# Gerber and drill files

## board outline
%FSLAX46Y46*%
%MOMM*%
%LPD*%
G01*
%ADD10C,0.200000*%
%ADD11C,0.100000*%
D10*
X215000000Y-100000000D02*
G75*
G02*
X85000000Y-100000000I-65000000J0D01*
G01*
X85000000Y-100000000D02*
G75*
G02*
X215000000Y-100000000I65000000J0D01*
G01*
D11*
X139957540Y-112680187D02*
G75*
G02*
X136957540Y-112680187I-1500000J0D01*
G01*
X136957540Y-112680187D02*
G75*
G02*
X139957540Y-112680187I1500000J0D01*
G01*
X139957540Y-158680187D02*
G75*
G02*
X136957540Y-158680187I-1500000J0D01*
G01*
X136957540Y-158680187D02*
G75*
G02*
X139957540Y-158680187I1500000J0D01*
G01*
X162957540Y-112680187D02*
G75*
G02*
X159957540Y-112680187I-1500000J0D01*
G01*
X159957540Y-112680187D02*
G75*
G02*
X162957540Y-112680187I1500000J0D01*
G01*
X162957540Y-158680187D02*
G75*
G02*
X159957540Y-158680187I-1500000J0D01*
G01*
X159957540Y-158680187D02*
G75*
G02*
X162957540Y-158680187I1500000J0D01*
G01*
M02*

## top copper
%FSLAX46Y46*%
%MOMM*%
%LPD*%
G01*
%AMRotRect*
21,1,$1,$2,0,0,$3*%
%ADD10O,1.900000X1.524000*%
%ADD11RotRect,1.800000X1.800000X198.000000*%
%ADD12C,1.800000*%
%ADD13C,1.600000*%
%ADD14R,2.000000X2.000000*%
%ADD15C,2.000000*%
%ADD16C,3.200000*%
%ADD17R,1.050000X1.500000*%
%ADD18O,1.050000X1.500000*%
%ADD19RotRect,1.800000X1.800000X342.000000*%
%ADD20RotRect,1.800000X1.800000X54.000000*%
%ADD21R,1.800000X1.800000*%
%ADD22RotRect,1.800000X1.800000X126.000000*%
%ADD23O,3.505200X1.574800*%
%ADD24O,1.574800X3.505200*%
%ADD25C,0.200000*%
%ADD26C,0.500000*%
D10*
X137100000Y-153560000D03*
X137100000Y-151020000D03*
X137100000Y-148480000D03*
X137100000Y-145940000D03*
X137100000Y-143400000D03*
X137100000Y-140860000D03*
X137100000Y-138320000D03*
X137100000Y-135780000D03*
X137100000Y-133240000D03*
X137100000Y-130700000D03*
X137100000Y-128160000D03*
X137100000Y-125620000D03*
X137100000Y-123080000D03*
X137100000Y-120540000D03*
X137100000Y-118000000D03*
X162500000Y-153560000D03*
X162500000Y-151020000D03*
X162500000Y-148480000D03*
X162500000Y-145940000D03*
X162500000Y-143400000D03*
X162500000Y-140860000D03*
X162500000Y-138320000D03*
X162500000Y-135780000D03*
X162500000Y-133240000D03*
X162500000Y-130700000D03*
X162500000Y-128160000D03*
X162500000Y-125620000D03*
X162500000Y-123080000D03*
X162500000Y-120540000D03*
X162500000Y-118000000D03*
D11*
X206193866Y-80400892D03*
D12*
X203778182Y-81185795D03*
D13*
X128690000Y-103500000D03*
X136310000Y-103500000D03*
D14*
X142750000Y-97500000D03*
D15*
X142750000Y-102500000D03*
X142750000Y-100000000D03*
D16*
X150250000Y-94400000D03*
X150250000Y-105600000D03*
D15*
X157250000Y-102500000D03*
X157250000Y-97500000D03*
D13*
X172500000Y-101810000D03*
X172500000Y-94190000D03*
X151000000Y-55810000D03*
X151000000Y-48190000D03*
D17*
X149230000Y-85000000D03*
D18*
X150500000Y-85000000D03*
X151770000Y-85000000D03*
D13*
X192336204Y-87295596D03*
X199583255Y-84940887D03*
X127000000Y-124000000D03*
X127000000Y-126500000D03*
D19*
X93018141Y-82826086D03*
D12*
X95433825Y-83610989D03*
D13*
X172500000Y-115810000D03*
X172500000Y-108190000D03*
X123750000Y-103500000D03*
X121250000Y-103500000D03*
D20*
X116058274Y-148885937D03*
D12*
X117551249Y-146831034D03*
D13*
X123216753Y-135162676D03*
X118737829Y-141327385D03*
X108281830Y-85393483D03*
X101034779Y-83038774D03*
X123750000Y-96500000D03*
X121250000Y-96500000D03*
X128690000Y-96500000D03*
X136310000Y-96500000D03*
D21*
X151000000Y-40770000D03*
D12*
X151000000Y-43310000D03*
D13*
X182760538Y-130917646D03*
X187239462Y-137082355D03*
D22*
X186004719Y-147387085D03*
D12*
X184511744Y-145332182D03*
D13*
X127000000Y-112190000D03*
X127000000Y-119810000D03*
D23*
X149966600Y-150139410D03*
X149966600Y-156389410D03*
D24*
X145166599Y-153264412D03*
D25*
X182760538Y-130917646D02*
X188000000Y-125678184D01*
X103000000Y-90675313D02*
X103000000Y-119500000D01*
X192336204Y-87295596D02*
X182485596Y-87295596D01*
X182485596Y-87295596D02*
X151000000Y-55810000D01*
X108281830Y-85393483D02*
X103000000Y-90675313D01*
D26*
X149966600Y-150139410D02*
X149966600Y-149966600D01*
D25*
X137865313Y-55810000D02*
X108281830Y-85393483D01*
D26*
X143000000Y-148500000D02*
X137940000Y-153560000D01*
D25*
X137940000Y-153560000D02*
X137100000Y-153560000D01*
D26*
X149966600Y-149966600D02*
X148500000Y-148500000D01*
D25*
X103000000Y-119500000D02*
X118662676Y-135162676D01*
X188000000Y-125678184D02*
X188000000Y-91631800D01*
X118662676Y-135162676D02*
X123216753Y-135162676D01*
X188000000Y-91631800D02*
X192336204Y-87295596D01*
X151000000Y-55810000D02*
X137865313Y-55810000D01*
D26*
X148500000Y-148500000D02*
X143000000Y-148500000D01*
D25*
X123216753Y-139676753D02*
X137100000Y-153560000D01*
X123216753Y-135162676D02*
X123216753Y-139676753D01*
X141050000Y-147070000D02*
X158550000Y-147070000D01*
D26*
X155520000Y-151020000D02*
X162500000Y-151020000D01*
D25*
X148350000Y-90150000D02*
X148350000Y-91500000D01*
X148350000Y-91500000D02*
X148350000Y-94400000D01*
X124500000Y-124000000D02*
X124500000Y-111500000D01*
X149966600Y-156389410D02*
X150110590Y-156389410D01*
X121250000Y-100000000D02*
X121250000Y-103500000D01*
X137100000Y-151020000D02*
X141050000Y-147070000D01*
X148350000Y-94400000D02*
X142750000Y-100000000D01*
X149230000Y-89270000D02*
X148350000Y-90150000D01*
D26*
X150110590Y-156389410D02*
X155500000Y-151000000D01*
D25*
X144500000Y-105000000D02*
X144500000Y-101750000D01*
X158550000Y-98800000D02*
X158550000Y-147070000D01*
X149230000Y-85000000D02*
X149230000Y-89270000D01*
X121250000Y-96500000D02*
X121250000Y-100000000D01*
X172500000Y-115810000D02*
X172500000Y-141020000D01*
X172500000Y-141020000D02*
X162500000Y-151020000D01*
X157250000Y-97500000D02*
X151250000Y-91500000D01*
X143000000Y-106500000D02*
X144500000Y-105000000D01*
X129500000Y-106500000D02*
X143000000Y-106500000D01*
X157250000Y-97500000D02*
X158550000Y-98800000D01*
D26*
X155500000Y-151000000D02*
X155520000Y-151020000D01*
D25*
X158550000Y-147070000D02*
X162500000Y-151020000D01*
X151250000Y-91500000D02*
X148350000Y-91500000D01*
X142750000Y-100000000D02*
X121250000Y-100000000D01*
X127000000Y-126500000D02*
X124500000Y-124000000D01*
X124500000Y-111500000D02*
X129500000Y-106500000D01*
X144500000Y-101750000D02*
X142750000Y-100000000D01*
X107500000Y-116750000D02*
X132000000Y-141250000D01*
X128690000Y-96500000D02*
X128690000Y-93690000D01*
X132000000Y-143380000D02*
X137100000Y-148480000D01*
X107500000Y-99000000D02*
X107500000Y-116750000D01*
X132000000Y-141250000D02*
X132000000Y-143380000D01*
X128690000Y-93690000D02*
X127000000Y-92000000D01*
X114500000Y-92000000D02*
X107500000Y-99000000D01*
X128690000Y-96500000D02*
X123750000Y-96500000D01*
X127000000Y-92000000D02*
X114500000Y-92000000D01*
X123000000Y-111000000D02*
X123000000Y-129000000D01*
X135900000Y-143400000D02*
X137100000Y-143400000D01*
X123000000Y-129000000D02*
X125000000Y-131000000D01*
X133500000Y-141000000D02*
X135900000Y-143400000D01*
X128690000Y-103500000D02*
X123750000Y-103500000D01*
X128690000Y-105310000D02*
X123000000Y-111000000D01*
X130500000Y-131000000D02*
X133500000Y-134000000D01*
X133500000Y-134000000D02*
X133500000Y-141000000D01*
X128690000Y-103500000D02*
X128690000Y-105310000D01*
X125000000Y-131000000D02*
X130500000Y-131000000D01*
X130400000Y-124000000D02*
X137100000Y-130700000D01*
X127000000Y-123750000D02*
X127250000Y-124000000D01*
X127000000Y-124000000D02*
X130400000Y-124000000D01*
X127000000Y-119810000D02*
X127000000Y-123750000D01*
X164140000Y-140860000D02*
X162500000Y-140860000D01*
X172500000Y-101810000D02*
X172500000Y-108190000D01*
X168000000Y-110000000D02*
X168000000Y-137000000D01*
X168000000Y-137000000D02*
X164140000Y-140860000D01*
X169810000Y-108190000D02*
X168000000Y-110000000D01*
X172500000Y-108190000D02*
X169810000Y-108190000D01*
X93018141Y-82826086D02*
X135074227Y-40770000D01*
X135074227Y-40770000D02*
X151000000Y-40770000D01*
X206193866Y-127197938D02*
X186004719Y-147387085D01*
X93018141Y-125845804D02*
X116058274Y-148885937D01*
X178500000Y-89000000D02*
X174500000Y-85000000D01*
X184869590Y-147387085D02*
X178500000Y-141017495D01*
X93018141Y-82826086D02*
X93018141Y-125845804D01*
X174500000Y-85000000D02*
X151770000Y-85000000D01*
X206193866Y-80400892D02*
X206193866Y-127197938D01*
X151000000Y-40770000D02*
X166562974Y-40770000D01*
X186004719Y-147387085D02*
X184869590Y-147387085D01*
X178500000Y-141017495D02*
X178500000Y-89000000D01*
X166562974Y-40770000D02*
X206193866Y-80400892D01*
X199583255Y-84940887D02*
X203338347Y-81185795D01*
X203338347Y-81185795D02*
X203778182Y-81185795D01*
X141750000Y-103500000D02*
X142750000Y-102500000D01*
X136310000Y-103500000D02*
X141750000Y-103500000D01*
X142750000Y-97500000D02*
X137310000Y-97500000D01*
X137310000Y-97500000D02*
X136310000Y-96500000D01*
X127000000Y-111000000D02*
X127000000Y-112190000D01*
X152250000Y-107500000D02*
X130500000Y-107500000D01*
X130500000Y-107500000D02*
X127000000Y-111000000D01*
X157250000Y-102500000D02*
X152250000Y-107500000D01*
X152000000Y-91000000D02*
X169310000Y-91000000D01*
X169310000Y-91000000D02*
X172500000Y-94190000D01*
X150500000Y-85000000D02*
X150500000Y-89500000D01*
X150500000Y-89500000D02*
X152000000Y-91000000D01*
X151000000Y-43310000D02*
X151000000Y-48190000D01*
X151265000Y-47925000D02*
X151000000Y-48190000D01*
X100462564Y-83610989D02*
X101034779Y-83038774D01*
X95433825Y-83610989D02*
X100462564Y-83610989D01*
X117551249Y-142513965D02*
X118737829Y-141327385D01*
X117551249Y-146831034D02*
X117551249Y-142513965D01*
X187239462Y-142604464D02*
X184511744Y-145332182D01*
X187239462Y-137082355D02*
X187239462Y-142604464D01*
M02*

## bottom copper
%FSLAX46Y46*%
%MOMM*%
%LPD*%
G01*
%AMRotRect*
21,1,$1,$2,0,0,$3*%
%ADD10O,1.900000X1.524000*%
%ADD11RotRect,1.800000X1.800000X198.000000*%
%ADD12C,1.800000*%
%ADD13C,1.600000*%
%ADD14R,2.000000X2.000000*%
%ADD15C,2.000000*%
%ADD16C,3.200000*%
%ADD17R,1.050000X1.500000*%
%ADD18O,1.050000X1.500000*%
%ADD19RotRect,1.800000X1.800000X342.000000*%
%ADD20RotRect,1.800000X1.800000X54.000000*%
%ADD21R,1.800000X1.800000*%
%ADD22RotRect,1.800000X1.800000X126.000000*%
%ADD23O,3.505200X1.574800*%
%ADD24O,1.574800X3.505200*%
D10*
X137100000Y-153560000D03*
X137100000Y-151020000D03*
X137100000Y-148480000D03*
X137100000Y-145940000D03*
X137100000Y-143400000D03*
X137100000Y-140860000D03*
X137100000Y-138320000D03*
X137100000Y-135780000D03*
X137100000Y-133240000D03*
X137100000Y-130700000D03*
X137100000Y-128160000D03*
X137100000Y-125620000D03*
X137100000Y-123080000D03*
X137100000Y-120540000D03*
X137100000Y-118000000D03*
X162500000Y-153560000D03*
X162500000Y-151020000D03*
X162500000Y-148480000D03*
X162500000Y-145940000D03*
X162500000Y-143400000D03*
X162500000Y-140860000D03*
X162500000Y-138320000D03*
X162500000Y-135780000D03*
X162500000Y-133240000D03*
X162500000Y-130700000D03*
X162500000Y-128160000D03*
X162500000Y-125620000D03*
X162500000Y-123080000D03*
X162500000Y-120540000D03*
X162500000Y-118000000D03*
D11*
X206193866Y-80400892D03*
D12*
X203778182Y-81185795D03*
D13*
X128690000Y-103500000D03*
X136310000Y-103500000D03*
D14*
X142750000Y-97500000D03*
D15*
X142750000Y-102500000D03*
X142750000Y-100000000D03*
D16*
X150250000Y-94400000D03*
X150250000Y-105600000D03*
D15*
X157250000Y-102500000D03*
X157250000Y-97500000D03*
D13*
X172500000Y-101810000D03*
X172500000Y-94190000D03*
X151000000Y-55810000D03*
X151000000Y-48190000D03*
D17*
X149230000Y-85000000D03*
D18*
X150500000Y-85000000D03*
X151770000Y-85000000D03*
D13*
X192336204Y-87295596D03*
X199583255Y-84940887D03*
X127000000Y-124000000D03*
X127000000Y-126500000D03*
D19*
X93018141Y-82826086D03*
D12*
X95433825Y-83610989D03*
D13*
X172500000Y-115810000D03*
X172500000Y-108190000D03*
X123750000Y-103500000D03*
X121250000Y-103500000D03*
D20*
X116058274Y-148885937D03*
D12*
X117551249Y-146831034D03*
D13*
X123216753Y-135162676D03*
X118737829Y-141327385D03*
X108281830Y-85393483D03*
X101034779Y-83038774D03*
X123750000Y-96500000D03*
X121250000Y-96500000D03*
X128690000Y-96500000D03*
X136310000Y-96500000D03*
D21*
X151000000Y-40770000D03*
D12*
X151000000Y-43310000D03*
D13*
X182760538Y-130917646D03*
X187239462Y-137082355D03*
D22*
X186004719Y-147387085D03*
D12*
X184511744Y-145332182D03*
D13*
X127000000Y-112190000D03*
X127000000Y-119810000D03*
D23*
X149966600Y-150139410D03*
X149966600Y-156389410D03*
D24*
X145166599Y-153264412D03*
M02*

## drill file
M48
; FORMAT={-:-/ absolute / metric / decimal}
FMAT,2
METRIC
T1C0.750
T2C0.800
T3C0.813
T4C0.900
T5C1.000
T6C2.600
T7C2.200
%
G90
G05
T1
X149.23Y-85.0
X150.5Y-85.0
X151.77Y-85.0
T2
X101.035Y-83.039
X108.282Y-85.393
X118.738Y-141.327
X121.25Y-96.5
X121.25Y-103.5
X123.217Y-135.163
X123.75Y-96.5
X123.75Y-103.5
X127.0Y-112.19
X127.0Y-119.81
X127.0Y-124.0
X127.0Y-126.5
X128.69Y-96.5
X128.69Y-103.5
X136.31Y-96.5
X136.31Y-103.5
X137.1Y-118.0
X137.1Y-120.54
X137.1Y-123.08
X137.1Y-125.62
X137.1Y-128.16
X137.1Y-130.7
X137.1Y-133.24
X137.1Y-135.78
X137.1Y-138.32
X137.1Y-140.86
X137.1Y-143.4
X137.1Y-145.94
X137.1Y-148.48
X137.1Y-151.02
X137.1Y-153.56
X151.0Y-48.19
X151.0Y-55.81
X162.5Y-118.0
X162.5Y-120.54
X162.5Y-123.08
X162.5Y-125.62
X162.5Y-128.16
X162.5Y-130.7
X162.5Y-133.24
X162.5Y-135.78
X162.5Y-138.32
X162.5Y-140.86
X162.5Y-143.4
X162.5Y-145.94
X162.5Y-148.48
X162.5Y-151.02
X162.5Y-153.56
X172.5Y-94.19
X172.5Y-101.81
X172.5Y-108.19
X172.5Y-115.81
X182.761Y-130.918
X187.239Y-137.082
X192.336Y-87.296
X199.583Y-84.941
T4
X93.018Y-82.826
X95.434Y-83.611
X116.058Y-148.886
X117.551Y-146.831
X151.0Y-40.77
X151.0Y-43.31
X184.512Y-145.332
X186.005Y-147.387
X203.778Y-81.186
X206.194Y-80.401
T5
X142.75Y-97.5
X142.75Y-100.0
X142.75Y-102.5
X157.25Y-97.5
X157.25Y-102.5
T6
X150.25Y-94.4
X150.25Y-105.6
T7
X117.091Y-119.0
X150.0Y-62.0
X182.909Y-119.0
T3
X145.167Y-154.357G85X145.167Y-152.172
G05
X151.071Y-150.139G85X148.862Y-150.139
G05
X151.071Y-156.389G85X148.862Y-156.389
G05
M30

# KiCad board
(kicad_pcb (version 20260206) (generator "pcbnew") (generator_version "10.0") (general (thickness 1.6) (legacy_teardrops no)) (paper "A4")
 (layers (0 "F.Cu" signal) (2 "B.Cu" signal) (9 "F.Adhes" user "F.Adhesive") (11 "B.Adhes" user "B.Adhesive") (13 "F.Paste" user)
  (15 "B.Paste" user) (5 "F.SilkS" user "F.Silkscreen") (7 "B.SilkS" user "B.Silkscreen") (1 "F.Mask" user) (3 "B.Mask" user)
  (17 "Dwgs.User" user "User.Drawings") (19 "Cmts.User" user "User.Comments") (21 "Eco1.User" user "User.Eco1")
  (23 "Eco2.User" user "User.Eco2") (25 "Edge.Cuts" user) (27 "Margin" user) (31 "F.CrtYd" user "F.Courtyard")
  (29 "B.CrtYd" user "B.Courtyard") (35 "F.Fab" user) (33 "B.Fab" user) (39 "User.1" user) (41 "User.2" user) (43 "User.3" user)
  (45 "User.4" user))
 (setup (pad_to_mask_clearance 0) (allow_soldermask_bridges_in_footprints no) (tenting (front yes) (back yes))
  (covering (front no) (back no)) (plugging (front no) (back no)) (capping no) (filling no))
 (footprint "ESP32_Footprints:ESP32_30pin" (layer "F.Cu") (at 149.02754 136.540187)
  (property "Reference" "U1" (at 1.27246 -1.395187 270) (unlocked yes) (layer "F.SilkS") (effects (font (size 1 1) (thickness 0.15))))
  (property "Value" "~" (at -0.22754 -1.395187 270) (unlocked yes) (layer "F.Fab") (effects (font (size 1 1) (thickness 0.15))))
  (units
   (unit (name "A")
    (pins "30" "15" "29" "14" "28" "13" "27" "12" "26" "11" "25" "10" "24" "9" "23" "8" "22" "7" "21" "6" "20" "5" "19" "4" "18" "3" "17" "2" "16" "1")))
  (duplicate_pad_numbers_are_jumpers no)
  (fp_circle (center -10.57 -23.86) (end -10.57 -22.36) (stroke (width 0.1) (type default)) (fill no) (layer "Edge.Cuts"))
  (fp_circle (center -10.57 22.14) (end -10.57 23.64) (stroke (width 0.1) (type default)) (fill no) (layer "Edge.Cuts"))
  (fp_circle (center 12.43 -23.86) (end 12.43 -22.36) (stroke (width 0.1) (type default)) (fill no) (layer "Edge.Cuts"))
  (fp_circle (center 12.43 22.14) (end 12.43 23.64) (stroke (width 0.1) (type default)) (fill no) (layer "Edge.Cuts"))
  (pad "1" thru_hole oval (at -11.92754 17.019813 270) (size 1.524 1.9) (drill 0.8) (layers "*.Cu" "*.Mask") (remove_unused_layers no)
   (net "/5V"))
  (pad "2" thru_hole oval (at -11.92754 14.479813 270) (size 1.524 1.9) (drill 0.8) (layers "*.Cu" "*.Mask") (remove_unused_layers no)
   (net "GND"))
  (pad "3" thru_hole oval (at -11.92754 11.939813 270) (size 1.524 1.9) (drill 0.8) (layers "*.Cu" "*.Mask") (remove_unused_layers no)
   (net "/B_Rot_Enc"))
  (pad "4" thru_hole oval (at -11.92754 9.399813 270) (size 1.524 1.9) (drill 0.8) (layers "*.Cu" "*.Mask") (remove_unused_layers no)
   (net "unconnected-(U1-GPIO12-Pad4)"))
  (pad "5" thru_hole oval (at -11.92754 6.859813 270) (size 1.524 1.9) (drill 0.8) (layers "*.Cu" "*.Mask") (remove_unused_layers no)
   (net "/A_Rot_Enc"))
  (pad "6" thru_hole oval (at -11.92754 4.319813 270) (size 1.524 1.9) (drill 0.8) (layers "*.Cu" "*.Mask") (remove_unused_layers no)
   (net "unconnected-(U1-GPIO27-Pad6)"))
  (pad "7" thru_hole oval (at -11.92754 1.779813 270) (size 1.524 1.9) (drill 0.8) (layers "*.Cu" "*.Mask") (remove_unused_layers no)
   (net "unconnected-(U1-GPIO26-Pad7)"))
  (pad "8" thru_hole oval (at -11.92754 -0.760187 270) (size 1.524 1.9) (drill 0.8) (layers "*.Cu" "*.Mask") (remove_unused_layers no)
   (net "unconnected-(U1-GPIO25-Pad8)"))
  (pad "9" thru_hole oval (at -11.92754 -3.300187 270) (size 1.524 1.9) (drill 0.8) (layers "*.Cu" "*.Mask") (remove_unused_layers no)
   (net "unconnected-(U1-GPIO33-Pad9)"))
  (pad "10" thru_hole oval (at -11.92754 -5.840187 270) (size 1.524 1.9) (drill 0.8) (layers "*.Cu" "*.Mask") (remove_unused_layers no)
   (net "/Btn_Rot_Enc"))
  (pad "11" thru_hole oval (at -11.92754 -8.380187 270) (size 1.524 1.9) (drill 0.8) (layers "*.Cu" "*.Mask") (remove_unused_layers no)
   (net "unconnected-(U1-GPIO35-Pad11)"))
  (pad "12" thru_hole oval (at -11.92754 -10.920187 270) (size 1.524 1.9) (drill 0.8) (layers "*.Cu" "*.Mask") (remove_unused_layers no)
   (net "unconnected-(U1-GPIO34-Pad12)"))
  (pad "13" thru_hole oval (at -11.92754 -13.460187 270) (size 1.524 1.9) (drill 0.8) (layers "*.Cu" "*.Mask") (remove_unused_layers no)
   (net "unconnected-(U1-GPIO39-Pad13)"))
  (pad "14" thru_hole oval (at -11.92754 -16.000187 270) (size 1.524 1.9) (drill 0.8) (layers "*.Cu" "*.Mask") (remove_unused_layers no)
   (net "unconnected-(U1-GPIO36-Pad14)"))
  (pad "15" thru_hole oval (at -11.92754 -18.540187 270) (size 1.524 1.9) (drill 0.8) (layers "*.Cu" "*.Mask") (remove_unused_layers no)
   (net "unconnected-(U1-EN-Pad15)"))
  (pad "16" thru_hole oval (at 13.47246 17.019813 270) (size 1.524 1.9) (drill 0.8) (layers "*.Cu" "*.Mask") (remove_unused_layers no)
   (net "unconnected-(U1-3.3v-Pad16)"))
  (pad "17" thru_hole oval (at 13.47246 14.479813 270) (size 1.524 1.9) (drill 0.8) (layers "*.Cu" "*.Mask") (remove_unused_layers no)
   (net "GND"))
  (pad "18" thru_hole oval (at 13.47246 11.939813 270) (size 1.524 1.9) (drill 0.8) (layers "*.Cu" "*.Mask") (remove_unused_layers no)
   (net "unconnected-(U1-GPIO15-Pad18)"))
  (pad "19" thru_hole oval (at 13.47246 9.399813 270) (size 1.524 1.9) (drill 0.8) (layers "*.Cu" "*.Mask") (remove_unused_layers no)
   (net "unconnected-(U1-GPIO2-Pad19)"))
  (pad "20" thru_hole oval (at 13.47246 6.859813 270) (size 1.524 1.9) (drill 0.8) (layers "*.Cu" "*.Mask" "Dwgs.User")
   (remove_unused_layers no) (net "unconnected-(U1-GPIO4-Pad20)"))
  (pad "21" thru_hole oval (at 13.47246 4.319813 270) (size 1.524 1.9) (drill 0.8) (layers "*.Cu" "*.Mask") (remove_unused_layers no)
   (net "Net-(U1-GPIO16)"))
  (pad "22" thru_hole oval (at 13.47246 1.779813 270) (size 1.524 1.9) (drill 0.8) (layers "*.Cu" "*.Mask") (remove_unused_layers no)
   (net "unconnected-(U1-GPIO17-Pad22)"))
  (pad "23" thru_hole oval (at 13.47246 -0.760187 270) (size 1.524 1.9) (drill 0.8) (layers "*.Cu" "*.Mask") (remove_unused_layers no)
   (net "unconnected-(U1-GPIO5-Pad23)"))
  (pad "24" thru_hole oval (at 13.47246 -3.300187 270) (size 1.524 1.9) (drill 0.8) (layers "*.Cu" "*.Mask") (remove_unused_layers no)
   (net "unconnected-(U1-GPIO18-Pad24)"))
  (pad "25" thru_hole oval (at 13.47246 -5.840187 270) (size 1.524 1.9) (drill 0.8) (layers "*.Cu" "*.Mask") (remove_unused_layers no)
   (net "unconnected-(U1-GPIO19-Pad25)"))
  (pad "26" thru_hole oval (at 13.47246 -8.380187 270) (size 1.524 1.9) (drill 0.8) (layers "*.Cu" "*.Mask") (remove_unused_layers no)
   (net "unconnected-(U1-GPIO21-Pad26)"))
  (pad "27" thru_hole oval (at 13.47246 -10.920187 270) (size 1.524 1.9) (drill 0.8) (layers "*.Cu" "*.Mask") (remove_unused_layers no)
   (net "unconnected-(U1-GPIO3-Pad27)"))
  (pad "28" thru_hole oval (at 13.47246 -13.460187 270) (size 1.524 1.9) (drill 0.8) (layers "*.Cu" "*.Mask") (remove_unused_layers no)
   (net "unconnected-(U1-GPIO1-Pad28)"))
  (pad "29" thru_hole oval (at 13.47246 -16.000187 270) (size 1.524 1.9) (drill 0.8) (layers "*.Cu" "*.Mask") (remove_unused_layers no)
   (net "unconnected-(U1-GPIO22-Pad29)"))
  (pad "30" thru_hole oval (at 13.47246 -18.540187 270) (size 1.524 1.9) (drill 0.8) (layers "*.Cu" "*.Mask") (remove_unused_layers no)
   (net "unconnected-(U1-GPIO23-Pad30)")))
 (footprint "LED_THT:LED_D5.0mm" (layer "F.Cu") (at 206.193866 80.400892 -162)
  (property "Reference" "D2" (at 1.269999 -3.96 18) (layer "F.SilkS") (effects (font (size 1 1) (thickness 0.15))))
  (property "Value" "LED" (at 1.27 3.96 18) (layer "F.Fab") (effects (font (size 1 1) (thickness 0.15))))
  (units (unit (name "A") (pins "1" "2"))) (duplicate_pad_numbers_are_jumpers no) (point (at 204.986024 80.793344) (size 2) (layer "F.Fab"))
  (pad "1" thru_hole rect (at 0 0 198) (size 1.8 1.8) (drill 0.9) (layers "*.Cu" "*.Mask") (remove_unused_layers no) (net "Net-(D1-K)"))
  (pad "2" thru_hole circle (at 2.54 0 198) (size 1.8 1.8) (drill 0.9) (layers "*.Cu" "*.Mask") (remove_unused_layers no) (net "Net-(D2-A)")))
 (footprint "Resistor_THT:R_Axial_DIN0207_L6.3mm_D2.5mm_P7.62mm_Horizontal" (layer "F.Cu") (at 128.69 103.5)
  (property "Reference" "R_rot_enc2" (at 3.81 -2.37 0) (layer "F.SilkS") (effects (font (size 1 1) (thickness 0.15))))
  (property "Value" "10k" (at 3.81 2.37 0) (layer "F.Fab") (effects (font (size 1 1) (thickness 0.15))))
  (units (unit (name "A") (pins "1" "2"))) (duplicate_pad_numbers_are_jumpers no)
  (pad "1" thru_hole circle (at 0 0) (size 1.6 1.6) (drill 0.8) (layers "*.Cu" "*.Mask") (remove_unused_layers no) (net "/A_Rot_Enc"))
  (pad "2" thru_hole circle (at 7.62 0) (size 1.6 1.6) (drill 0.8) (layers "*.Cu" "*.Mask") (remove_unused_layers no)
   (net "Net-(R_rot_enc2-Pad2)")))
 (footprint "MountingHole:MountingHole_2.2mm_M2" (layer "F.Cu") (at 182.909 119)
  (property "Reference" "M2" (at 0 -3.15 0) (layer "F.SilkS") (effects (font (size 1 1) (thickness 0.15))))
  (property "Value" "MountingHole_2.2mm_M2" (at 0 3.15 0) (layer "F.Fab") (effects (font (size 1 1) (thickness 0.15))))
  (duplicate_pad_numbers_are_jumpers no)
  (pad "" np_thru_hole circle (at 0 0) (size 2.2 2.2) (drill 2.2) (layers "*.Cu" "*.Mask")))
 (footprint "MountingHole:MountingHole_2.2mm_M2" (layer "F.Cu") (at 117.091 119)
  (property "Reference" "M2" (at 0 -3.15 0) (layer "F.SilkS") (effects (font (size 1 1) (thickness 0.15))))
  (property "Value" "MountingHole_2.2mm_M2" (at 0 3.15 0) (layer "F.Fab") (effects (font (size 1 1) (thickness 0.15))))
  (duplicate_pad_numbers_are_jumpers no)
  (pad "" np_thru_hole circle (at 0 0) (size 2.2 2.2) (drill 2.2) (layers "*.Cu" "*.Mask")))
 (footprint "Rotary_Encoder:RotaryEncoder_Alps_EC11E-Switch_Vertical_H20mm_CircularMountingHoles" (layer "F.Cu") (at 142.75 97.5)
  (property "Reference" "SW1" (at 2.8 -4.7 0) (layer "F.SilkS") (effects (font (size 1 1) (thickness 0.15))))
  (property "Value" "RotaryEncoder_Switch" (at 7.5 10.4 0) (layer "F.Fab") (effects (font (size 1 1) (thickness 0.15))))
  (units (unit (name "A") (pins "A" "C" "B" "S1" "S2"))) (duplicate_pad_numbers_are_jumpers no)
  (pad "A" thru_hole rect (at 0 0) (size 2 2) (drill 1) (layers "*.Cu" "*.Mask") (remove_unused_layers no) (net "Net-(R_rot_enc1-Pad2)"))
  (pad "B" thru_hole circle (at 0 5) (size 2 2) (drill 1) (layers "*.Cu" "*.Mask") (remove_unused_layers no) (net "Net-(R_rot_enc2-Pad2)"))
  (pad "C" thru_hole circle (at 0 2.5) (size 2 2) (drill 1) (layers "*.Cu" "*.Mask") (remove_unused_layers no) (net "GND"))
  (pad "MP" thru_hole circle (at 7.5 -3.1) (size 3.2 3.2) (drill 2.6) (layers "*.Cu" "*.Mask") (remove_unused_layers no))
  (pad "MP" thru_hole circle (at 7.5 8.1) (size 3.2 3.2) (drill 2.6) (layers "*.Cu" "*.Mask") (remove_unused_layers no))
  (pad "S1" thru_hole circle (at 14.5 5) (size 2 2) (drill 1) (layers "*.Cu" "*.Mask") (remove_unused_layers no) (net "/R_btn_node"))
  (pad "S2" thru_hole circle (at 14.5 0) (size 2 2) (drill 1) (layers "*.Cu" "*.Mask") (remove_unused_layers no) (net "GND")))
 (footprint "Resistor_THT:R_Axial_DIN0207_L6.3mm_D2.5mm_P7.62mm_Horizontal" (layer "F.Cu") (at 172.5 101.81 90)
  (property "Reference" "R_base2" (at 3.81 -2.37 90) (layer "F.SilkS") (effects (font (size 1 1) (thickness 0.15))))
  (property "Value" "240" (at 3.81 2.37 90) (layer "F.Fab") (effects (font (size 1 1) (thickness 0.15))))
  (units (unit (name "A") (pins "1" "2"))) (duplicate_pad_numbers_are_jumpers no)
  (pad "1" thru_hole circle (at 0 0 90) (size 1.6 1.6) (drill 0.8) (layers "*.Cu" "*.Mask") (remove_unused_layers no)
   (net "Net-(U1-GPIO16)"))
  (pad "2" thru_hole circle (at 7.62 0 90) (size 1.6 1.6) (drill 0.8) (layers "*.Cu" "*.Mask") (remove_unused_layers no) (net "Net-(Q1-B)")))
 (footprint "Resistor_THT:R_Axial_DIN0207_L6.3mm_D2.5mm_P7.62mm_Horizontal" (layer "F.Cu") (at 151 55.81 90)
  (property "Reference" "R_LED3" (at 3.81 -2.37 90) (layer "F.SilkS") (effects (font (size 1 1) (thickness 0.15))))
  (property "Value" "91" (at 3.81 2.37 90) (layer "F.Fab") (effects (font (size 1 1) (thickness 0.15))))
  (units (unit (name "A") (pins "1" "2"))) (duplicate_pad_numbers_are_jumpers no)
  (pad "1" thru_hole circle (at 0 0 90) (size 1.6 1.6) (drill 0.8) (layers "*.Cu" "*.Mask") (remove_unused_layers no) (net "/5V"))
  (pad "2" thru_hole circle (at 7.62 0 90) (size 1.6 1.6) (drill 0.8) (layers "*.Cu" "*.Mask") (remove_unused_layers no) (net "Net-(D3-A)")))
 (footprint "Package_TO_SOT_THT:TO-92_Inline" (layer "F.Cu") (at 149.23 85)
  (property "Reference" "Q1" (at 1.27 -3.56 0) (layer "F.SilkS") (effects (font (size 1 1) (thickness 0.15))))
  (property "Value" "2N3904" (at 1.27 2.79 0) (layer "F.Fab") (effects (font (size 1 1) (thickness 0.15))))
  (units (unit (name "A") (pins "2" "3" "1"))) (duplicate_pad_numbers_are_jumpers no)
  (pad "1" thru_hole rect (at 0 0) (size 1.05 1.5) (drill 0.75) (layers "*.Cu" "*.Mask") (remove_unused_layers no) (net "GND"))
  (pad "2" thru_hole oval (at 1.27 0) (size 1.05 1.5) (drill 0.75) (layers "*.Cu" "*.Mask") (remove_unused_layers no) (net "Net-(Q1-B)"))
  (pad "3" thru_hole oval (at 2.54 0) (size 1.05 1.5) (drill 0.75) (layers "*.Cu" "*.Mask") (remove_unused_layers no) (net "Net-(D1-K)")))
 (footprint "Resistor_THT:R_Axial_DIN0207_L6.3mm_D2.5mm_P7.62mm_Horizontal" (layer "F.Cu") (at 192.336204 87.295596 18)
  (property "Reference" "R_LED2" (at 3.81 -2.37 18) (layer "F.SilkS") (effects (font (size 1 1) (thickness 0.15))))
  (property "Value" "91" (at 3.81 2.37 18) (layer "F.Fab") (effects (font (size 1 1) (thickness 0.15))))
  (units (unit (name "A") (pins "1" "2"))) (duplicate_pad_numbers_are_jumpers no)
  (pad "1" thru_hole circle (at 0 0 18) (size 1.6 1.6) (drill 0.8) (layers "*.Cu" "*.Mask") (remove_unused_layers no) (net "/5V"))
  (pad "2" thru_hole circle (at 7.62 0.000001 18) (size 1.6 1.6) (drill 0.8) (layers "*.Cu" "*.Mask") (remove_unused_layers no)
   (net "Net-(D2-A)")))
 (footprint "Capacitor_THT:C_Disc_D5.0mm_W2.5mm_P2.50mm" (layer "F.Cu") (at 127 124 -90)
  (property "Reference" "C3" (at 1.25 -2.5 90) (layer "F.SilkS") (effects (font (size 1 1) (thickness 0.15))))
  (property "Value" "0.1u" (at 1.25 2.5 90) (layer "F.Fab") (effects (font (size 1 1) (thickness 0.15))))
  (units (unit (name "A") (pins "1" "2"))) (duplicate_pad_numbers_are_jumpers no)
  (pad "1" thru_hole circle (at 0 0 270) (size 1.6 1.6) (drill 0.8) (layers "*.Cu" "*.Mask") (remove_unused_layers no) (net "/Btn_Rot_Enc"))
  (pad "2" thru_hole circle (at 2.5 0 270) (size 1.6 1.6) (drill 0.8) (layers "*.Cu" "*.Mask") (remove_unused_layers no) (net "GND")))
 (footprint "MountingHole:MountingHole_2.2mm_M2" (layer "F.Cu") (at 150 62)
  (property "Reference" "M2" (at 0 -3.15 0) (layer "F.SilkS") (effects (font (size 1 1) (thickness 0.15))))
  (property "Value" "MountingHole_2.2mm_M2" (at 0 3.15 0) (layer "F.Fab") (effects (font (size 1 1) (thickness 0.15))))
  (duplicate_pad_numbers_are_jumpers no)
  (pad "" np_thru_hole circle (at 0 0) (size 2.2 2.2) (drill 2.2) (layers "*.Cu" "*.Mask")))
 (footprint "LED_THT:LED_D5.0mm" (layer "F.Cu") (at 93.018141 82.826086 -18)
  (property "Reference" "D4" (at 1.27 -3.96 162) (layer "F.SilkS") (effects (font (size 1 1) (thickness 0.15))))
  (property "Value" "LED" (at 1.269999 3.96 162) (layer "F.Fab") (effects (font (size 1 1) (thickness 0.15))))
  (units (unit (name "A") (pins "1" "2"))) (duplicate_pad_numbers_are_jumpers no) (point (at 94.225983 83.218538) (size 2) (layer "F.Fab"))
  (pad "1" thru_hole rect (at 0 0 342) (size 1.8 1.8) (drill 0.9) (layers "*.Cu" "*.Mask") (remove_unused_layers no) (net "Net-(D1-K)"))
  (pad "2" thru_hole circle (at 2.54 0 342) (size 1.8 1.8) (drill 0.9) (layers "*.Cu" "*.Mask") (remove_unused_layers no) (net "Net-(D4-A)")))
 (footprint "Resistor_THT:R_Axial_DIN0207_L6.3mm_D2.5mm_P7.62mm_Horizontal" (layer "F.Cu") (at 172.5 115.81 90)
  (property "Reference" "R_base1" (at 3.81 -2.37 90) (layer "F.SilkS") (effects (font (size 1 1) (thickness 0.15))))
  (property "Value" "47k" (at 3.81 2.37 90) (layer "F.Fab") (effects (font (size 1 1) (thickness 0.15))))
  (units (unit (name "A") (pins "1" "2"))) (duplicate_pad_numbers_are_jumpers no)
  (pad "1" thru_hole circle (at 0 0 90) (size 1.6 1.6) (drill 0.8) (layers "*.Cu" "*.Mask") (remove_unused_layers no) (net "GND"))
  (pad "2" thru_hole circle (at 7.62 0 90) (size 1.6 1.6) (drill 0.8) (layers "*.Cu" "*.Mask") (remove_unused_layers no)
   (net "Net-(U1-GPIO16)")))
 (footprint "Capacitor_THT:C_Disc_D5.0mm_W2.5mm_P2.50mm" (layer "F.Cu") (at 123.75 103.5 180)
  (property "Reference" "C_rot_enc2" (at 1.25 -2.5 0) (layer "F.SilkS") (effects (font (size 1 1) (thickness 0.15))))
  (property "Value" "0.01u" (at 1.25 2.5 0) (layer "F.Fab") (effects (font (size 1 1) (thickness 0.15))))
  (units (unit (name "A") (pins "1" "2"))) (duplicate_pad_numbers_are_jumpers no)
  (pad "1" thru_hole circle (at 0 0 180) (size 1.6 1.6) (drill 0.8) (layers "*.Cu" "*.Mask") (remove_unused_layers no) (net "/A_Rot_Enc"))
  (pad "2" thru_hole circle (at 2.5 0 180) (size 1.6 1.6) (drill 0.8) (layers "*.Cu" "*.Mask") (remove_unused_layers no) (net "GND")))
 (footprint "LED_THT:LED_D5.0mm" (layer "F.Cu") (at 116.058274 148.885937 54)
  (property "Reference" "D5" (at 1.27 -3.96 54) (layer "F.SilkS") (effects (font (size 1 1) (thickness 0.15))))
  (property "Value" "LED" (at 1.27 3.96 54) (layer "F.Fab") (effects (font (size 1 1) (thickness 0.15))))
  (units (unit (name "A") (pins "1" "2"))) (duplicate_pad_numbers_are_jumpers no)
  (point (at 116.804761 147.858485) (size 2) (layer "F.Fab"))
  (pad "1" thru_hole rect (at 0 0 54) (size 1.8 1.8) (drill 0.9) (layers "*.Cu" "*.Mask") (remove_unused_layers no) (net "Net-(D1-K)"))
  (pad "2" thru_hole circle (at 2.54 0 54) (size 1.8 1.8) (drill 0.9) (layers "*.Cu" "*.Mask") (remove_unused_layers no) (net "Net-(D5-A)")))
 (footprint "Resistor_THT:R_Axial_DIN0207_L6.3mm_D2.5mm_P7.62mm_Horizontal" (layer "F.Cu") (at 123.216753 135.162676 -126)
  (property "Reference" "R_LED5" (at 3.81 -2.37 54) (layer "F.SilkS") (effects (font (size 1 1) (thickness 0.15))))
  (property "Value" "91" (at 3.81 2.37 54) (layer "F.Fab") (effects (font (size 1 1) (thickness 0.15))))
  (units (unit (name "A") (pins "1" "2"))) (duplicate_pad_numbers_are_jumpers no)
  (pad "1" thru_hole circle (at 0 0 234) (size 1.6 1.6) (drill 0.8) (layers "*.Cu" "*.Mask") (remove_unused_layers no) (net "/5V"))
  (pad "2" thru_hole circle (at 7.62 0.000001 234) (size 1.6 1.6) (drill 0.8) (layers "*.Cu" "*.Mask") (remove_unused_layers no)
   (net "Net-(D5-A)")))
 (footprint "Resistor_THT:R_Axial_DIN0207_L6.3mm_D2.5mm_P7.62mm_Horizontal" (layer "F.Cu") (at 108.28183 85.393483 162)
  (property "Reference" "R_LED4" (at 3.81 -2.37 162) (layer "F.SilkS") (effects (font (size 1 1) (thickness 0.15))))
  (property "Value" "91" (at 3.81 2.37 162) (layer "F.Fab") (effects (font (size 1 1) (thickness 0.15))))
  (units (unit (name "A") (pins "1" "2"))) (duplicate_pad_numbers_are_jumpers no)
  (pad "1" thru_hole circle (at 0 0 162) (size 1.6 1.6) (drill 0.8) (layers "*.Cu" "*.Mask") (remove_unused_layers no) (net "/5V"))
  (pad "2" thru_hole circle (at 7.62 -0.000001 162) (size 1.6 1.6) (drill 0.8) (layers "*.Cu" "*.Mask") (remove_unused_layers no)
   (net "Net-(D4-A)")))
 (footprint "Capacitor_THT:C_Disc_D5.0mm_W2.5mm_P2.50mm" (layer "F.Cu") (at 123.75 96.5 180)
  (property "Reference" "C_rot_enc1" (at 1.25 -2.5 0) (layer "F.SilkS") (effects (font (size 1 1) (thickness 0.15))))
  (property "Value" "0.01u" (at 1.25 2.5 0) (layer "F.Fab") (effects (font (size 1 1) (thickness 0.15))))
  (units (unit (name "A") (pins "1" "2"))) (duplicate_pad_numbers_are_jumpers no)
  (pad "1" thru_hole circle (at 0 0 180) (size 1.6 1.6) (drill 0.8) (layers "*.Cu" "*.Mask") (remove_unused_layers no) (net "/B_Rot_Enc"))
  (pad "2" thru_hole circle (at 2.5 0 180) (size 1.6 1.6) (drill 0.8) (layers "*.Cu" "*.Mask") (remove_unused_layers no) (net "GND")))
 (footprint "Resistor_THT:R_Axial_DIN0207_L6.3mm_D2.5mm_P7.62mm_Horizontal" (layer "F.Cu") (at 128.69 96.5)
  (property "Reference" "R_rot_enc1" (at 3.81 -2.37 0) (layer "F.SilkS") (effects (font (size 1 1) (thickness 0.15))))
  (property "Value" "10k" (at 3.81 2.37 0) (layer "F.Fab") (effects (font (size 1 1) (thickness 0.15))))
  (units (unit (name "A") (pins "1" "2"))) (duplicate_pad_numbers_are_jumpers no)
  (pad "1" thru_hole circle (at 0 0) (size 1.6 1.6) (drill 0.8) (layers "*.Cu" "*.Mask") (remove_unused_layers no) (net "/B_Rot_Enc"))
  (pad "2" thru_hole circle (at 7.62 0) (size 1.6 1.6) (drill 0.8) (layers "*.Cu" "*.Mask") (remove_unused_layers no)
   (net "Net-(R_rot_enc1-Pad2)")))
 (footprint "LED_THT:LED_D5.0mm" (layer "F.Cu") (at 151 40.77 -90)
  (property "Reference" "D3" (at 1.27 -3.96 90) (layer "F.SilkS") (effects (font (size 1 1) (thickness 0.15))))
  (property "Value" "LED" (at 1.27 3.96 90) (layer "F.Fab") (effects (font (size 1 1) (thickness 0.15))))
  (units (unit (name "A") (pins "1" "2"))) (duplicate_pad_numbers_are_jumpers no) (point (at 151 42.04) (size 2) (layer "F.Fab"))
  (pad "1" thru_hole rect (at 0 0 270) (size 1.8 1.8) (drill 0.9) (layers "*.Cu" "*.Mask") (remove_unused_layers no) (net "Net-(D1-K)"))
  (pad "2" thru_hole circle (at 2.54 0 270) (size 1.8 1.8) (drill 0.9) (layers "*.Cu" "*.Mask") (remove_unused_layers no) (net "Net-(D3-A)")))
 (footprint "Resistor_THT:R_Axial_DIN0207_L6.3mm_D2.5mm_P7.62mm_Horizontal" (layer "F.Cu") (at 182.760538 130.917646 -54)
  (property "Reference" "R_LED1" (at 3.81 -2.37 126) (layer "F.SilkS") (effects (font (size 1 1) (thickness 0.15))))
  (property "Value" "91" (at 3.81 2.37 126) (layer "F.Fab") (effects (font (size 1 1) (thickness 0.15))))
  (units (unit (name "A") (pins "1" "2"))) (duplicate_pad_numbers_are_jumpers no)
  (pad "1" thru_hole circle (at 0 0 306) (size 1.6 1.6) (drill 0.8) (layers "*.Cu" "*.Mask") (remove_unused_layers no) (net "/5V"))
  (pad "2" thru_hole circle (at 7.62 -0.000001 306) (size 1.6 1.6) (drill 0.8) (layers "*.Cu" "*.Mask") (remove_unused_layers no)
   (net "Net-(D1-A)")))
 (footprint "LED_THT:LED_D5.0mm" (layer "F.Cu") (at 186.004719 147.387085 126)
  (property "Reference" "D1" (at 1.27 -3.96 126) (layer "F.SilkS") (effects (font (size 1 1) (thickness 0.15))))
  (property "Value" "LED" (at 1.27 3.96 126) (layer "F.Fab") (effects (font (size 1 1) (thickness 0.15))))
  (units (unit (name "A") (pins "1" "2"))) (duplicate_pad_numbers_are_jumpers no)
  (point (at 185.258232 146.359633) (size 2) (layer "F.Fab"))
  (pad "1" thru_hole rect (at 0 0 126) (size 1.8 1.8) (drill 0.9) (layers "*.Cu" "*.Mask") (remove_unused_layers no) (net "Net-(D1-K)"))
  (pad "2" thru_hole circle (at 2.54 0 126) (size 1.8 1.8) (drill 0.9) (layers "*.Cu" "*.Mask") (remove_unused_layers no) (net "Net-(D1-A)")))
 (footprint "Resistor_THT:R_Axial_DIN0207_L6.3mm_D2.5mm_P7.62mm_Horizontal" (layer "F.Cu") (at 127 112.19 -90)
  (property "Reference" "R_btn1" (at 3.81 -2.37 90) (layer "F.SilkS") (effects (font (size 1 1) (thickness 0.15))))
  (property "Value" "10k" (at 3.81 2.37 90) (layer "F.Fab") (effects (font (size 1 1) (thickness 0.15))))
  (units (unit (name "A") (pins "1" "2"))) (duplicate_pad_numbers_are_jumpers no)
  (pad "1" thru_hole circle (at 0 0 270) (size 1.6 1.6) (drill 0.8) (layers "*.Cu" "*.Mask") (remove_unused_layers no) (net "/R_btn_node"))
  (pad "2" thru_hole circle (at 7.62 0 270) (size 1.6 1.6) (drill 0.8) (layers "*.Cu" "*.Mask") (remove_unused_layers no)
   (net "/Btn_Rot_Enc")))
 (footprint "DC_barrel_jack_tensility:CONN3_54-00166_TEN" (layer "B.Cu") (at 149.9666 150.13941 180)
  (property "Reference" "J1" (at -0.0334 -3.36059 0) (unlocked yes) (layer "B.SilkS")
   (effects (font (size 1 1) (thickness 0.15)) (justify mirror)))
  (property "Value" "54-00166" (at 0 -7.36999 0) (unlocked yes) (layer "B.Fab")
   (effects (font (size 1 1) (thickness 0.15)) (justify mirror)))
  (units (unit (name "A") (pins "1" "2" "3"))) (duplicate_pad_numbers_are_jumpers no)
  (pad "1" thru_hole oval (at 0 0 180) (size 3.5052 1.5748) (drill oval 3.0226 0.8128) (layers "*.Cu" "*.Mask") (remove_unused_layers no)
   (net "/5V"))
  (pad "2" thru_hole oval (at 0 -6.25 180) (size 3.5052 1.5748) (drill oval 3.0226 0.8128) (layers "*.Cu" "*.Mask")
   (remove_unused_layers no) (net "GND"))
  (pad "3" thru_hole oval (at 4.800001 -3.125002 90) (size 3.5052 1.5748) (drill oval 2.9972 0.8128) (layers "*.Cu" "*.Mask")
   (remove_unused_layers no) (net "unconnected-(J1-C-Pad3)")))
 (gr_circle (center 150 100) (end 215 100) (stroke (width 0.2) (type solid)) (fill no) (layer "Edge.Cuts"))
 (segment (start 182.760538 130.917646) (end 188 125.678184) (width 0.2) (layer "F.Cu") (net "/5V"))
 (segment (start 103 90.675313) (end 103 119.5) (width 0.2) (layer "F.Cu") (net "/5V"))
 (segment (start 192.336204 87.295596) (end 182.485596 87.295596) (width 0.2) (layer "F.Cu") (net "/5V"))
 (segment (start 182.485596 87.295596) (end 151 55.81) (width 0.2) (layer "F.Cu") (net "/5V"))
 (segment (start 108.28183 85.393483) (end 103 90.675313) (width 0.2) (layer "F.Cu") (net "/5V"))
 (segment (start 149.9666 150.13941) (end 149.9666 149.9666) (width 0.5) (layer "F.Cu") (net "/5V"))
 (segment (start 137.865313 55.81) (end 108.28183 85.393483) (width 0.2) (layer "F.Cu") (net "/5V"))
 (segment (start 143 148.5) (end 137.94 153.56) (width 0.5) (layer "F.Cu") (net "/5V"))
 (segment (start 137.94 153.56) (end 137.1 153.56) (width 0.2) (layer "F.Cu") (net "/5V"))
 (segment (start 149.9666 149.9666) (end 148.5 148.5) (width 0.5) (layer "F.Cu") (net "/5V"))
 (segment (start 103 119.5) (end 118.662676 135.162676) (width 0.2) (layer "F.Cu") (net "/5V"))
 (segment (start 188 125.678184) (end 188 91.6318) (width 0.2) (layer "F.Cu") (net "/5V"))
 (segment (start 118.662676 135.162676) (end 123.216753 135.162676) (width 0.2) (layer "F.Cu") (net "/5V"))
 (segment (start 188 91.6318) (end 192.336204 87.295596) (width 0.2) (layer "F.Cu") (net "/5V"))
 (segment (start 151 55.81) (end 137.865313 55.81) (width 0.2) (layer "F.Cu") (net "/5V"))
 (segment (start 148.5 148.5) (end 143 148.5) (width 0.5) (layer "F.Cu") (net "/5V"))
 (segment (start 123.216753 139.676753) (end 137.1 153.56) (width 0.2) (layer "F.Cu") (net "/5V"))
 (segment (start 123.216753 135.162676) (end 123.216753 139.676753) (width 0.2) (layer "F.Cu") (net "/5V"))
 (segment (start 141.05 147.07) (end 158.55 147.07) (width 0.2) (layer "F.Cu") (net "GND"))
 (segment (start 155.52 151.02) (end 162.5 151.02) (width 0.5) (layer "F.Cu") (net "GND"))
 (segment (start 148.35 90.15) (end 148.35 91.5) (width 0.2) (layer "F.Cu") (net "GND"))
 (segment (start 148.35 91.5) (end 148.35 94.4) (width 0.2) (layer "F.Cu") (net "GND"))
 (segment (start 124.5 124) (end 124.5 111.5) (width 0.2) (layer "F.Cu") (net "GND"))
 (segment (start 149.9666 156.38941) (end 150.11059 156.38941) (width 0.2) (layer "F.Cu") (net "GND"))
 (segment (start 121.25 100) (end 121.25 103.5) (width 0.2) (layer "F.Cu") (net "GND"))
 (segment (start 137.1 151.02) (end 141.05 147.07) (width 0.2) (layer "F.Cu") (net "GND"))
 (segment (start 148.35 94.4) (end 142.75 100) (width 0.2) (layer "F.Cu") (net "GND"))
 (segment (start 149.23 89.27) (end 148.35 90.15) (width 0.2) (layer "F.Cu") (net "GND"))
 (segment (start 150.11059 156.38941) (end 155.5 151) (width 0.5) (layer "F.Cu") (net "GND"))
 (segment (start 144.5 105) (end 144.5 101.75) (width 0.2) (layer "F.Cu") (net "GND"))
 (segment (start 158.55 98.8) (end 158.55 147.07) (width 0.2) (layer "F.Cu") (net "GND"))
 (segment (start 149.23 85) (end 149.23 89.27) (width 0.2) (layer "F.Cu") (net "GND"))
 (segment (start 121.25 96.5) (end 121.25 100) (width 0.2) (layer "F.Cu") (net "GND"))
 (segment (start 172.5 115.81) (end 172.5 141.02) (width 0.2) (layer "F.Cu") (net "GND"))
 (segment (start 172.5 141.02) (end 162.5 151.02) (width 0.2) (layer "F.Cu") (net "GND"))
 (segment (start 157.25 97.5) (end 151.25 91.5) (width 0.2) (layer "F.Cu") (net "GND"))
 (segment (start 143 106.5) (end 144.5 105) (width 0.2) (layer "F.Cu") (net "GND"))
 (segment (start 129.5 106.5) (end 143 106.5) (width 0.2) (layer "F.Cu") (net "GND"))
 (segment (start 157.25 97.5) (end 158.55 98.8) (width 0.2) (layer "F.Cu") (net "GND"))
 (segment (start 155.5 151) (end 155.52 151.02) (width 0.5) (layer "F.Cu") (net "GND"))
 (segment (start 158.55 147.07) (end 162.5 151.02) (width 0.2) (layer "F.Cu") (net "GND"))
 (segment (start 151.25 91.5) (end 148.35 91.5) (width 0.2) (layer "F.Cu") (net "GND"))
 (segment (start 142.75 100) (end 121.25 100) (width 0.2) (layer "F.Cu") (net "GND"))
 (segment (start 127 126.5) (end 124.5 124) (width 0.2) (layer "F.Cu") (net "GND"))
 (segment (start 124.5 111.5) (end 129.5 106.5) (width 0.2) (layer "F.Cu") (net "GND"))
 (segment (start 144.5 101.75) (end 142.75 100) (width 0.2) (layer "F.Cu") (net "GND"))
 (segment (start 107.5 116.75) (end 132 141.25) (width 0.2) (layer "F.Cu") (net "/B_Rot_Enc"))
 (segment (start 128.69 96.5) (end 128.69 93.69) (width 0.2) (layer "F.Cu") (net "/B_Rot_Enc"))
 (segment (start 132 143.38) (end 137.1 148.48) (width 0.2) (layer "F.Cu") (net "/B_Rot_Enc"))
 (segment (start 107.5 99) (end 107.5 116.75) (width 0.2) (layer "F.Cu") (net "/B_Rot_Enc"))
 (segment (start 132 141.25) (end 132 143.38) (width 0.2) (layer "F.Cu") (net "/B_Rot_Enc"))
 (segment (start 128.69 93.69) (end 127 92) (width 0.2) (layer "F.Cu") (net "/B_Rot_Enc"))
 (segment (start 114.5 92) (end 107.5 99) (width 0.2) (layer "F.Cu") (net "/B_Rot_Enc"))
 (segment (start 128.69 96.5) (end 123.75 96.5) (width 0.2) (layer "F.Cu") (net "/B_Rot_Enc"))
 (segment (start 127 92) (end 114.5 92) (width 0.2) (layer "F.Cu") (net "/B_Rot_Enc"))
 (segment (start 123 111) (end 123 129) (width 0.2) (layer "F.Cu") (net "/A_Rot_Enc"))
 (segment (start 135.9 143.4) (end 137.1 143.4) (width 0.2) (layer "F.Cu") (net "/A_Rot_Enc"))
 (segment (start 123 129) (end 125 131) (width 0.2) (layer "F.Cu") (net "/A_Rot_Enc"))
 (segment (start 133.5 141) (end 135.9 143.4) (width 0.2) (layer "F.Cu") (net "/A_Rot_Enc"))
 (segment (start 128.69 103.5) (end 123.75 103.5) (width 0.2) (layer "F.Cu") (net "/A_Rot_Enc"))
 (segment (start 128.69 105.31) (end 123 111) (width 0.2) (layer "F.Cu") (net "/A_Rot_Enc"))
 (segment (start 130.5 131) (end 133.5 134) (width 0.2) (layer "F.Cu") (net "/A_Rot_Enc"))
 (segment (start 133.5 134) (end 133.5 141) (width 0.2) (layer "F.Cu") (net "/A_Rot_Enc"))
 (segment (start 128.69 103.5) (end 128.69 105.31) (width 0.2) (layer "F.Cu") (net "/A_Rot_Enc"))
 (segment (start 125 131) (end 130.5 131) (width 0.2) (layer "F.Cu") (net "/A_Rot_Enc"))
 (segment (start 130.4 124) (end 137.1 130.7) (width 0.2) (layer "F.Cu") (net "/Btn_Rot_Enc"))
 (segment (start 127 123.75) (end 127.25 124) (width 0.2) (layer "F.Cu") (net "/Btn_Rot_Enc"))
 (segment (start 127 124) (end 130.4 124) (width 0.2) (layer "F.Cu") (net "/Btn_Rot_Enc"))
 (segment (start 127 119.81) (end 127 123.75) (width 0.2) (layer "F.Cu") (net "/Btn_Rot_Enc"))
 (segment (start 164.14 140.86) (end 162.5 140.86) (width 0.2) (layer "F.Cu") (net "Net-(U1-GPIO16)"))
 (segment (start 172.5 101.81) (end 172.5 108.19) (width 0.2) (layer "F.Cu") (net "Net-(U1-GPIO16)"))
 (segment (start 168 110) (end 168 137) (width 0.2) (layer "F.Cu") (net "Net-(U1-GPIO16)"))
 (segment (start 168 137) (end 164.14 140.86) (width 0.2) (layer "F.Cu") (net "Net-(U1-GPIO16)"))
 (segment (start 169.81 108.19) (end 168 110) (width 0.2) (layer "F.Cu") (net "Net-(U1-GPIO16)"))
 (segment (start 172.5 108.19) (end 169.81 108.19) (width 0.2) (layer "F.Cu") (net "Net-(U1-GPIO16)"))
 (segment (start 93.018141 82.826086) (end 135.074227 40.77) (width 0.2) (layer "F.Cu") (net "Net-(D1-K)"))
 (segment (start 135.074227 40.77) (end 151 40.77) (width 0.2) (layer "F.Cu") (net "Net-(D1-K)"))
 (segment (start 206.193866 127.197938) (end 186.004719 147.387085) (width 0.2) (layer "F.Cu") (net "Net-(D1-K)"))
 (segment (start 93.018141 125.845804) (end 116.058274 148.885937) (width 0.2) (layer "F.Cu") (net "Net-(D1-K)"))
 (segment (start 178.5 89) (end 174.5 85) (width 0.2) (layer "F.Cu") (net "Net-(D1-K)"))
 (segment (start 184.86959 147.387085) (end 178.5 141.017495) (width 0.2) (layer "F.Cu") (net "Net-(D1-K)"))
 (segment (start 93.018141 82.826086) (end 93.018141 125.845804) (width 0.2) (layer "F.Cu") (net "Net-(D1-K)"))
 (segment (start 174.5 85) (end 151.77 85) (width 0.2) (layer "F.Cu") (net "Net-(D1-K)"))
 (segment (start 206.193866 80.400892) (end 206.193866 127.197938) (width 0.2) (layer "F.Cu") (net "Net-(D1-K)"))
 (segment (start 151 40.77) (end 166.562974 40.77) (width 0.2) (layer "F.Cu") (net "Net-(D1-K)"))
 (segment (start 186.004719 147.387085) (end 184.86959 147.387085) (width 0.2) (layer "F.Cu") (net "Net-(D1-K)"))
 (segment (start 178.5 141.017495) (end 178.5 89) (width 0.2) (layer "F.Cu") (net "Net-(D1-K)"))
 (segment (start 166.562974 40.77) (end 206.193866 80.400892) (width 0.2) (layer "F.Cu") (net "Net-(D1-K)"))
 (segment (start 199.583255 84.940887) (end 203.338347 81.185795) (width 0.2) (layer "F.Cu") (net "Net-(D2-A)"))
 (segment (start 203.338347 81.185795) (end 203.778182 81.185795) (width 0.2) (layer "F.Cu") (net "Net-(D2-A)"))
 (segment (start 141.75 103.5) (end 142.75 102.5) (width 0.2) (layer "F.Cu") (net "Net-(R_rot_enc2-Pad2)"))
 (segment (start 136.31 103.5) (end 141.75 103.5) (width 0.2) (layer "F.Cu") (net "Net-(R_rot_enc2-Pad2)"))
 (segment (start 142.75 97.5) (end 137.31 97.5) (width 0.2) (layer "F.Cu") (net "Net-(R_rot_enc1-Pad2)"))
 (segment (start 137.31 97.5) (end 136.31 96.5) (width 0.2) (layer "F.Cu") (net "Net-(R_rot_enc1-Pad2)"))
 (segment (start 127 111) (end 127 112.19) (width 0.2) (layer "F.Cu") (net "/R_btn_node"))
 (segment (start 152.25 107.5) (end 130.5 107.5) (width 0.2) (layer "F.Cu") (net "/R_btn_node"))
 (segment (start 130.5 107.5) (end 127 111) (width 0.2) (layer "F.Cu") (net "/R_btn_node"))
 (segment (start 157.25 102.5) (end 152.25 107.5) (width 0.2) (layer "F.Cu") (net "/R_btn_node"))
 (segment (start 152 91) (end 169.31 91) (width 0.2) (layer "F.Cu") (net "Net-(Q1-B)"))
 (segment (start 169.31 91) (end 172.5 94.19) (width 0.2) (layer "F.Cu") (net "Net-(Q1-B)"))
 (segment (start 150.5 85) (end 150.5 89.5) (width 0.2) (layer "F.Cu") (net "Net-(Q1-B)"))
 (segment (start 150.5 89.5) (end 152 91) (width 0.2) (layer "F.Cu") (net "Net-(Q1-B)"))
 (segment (start 151 43.31) (end 151 48.19) (width 0.2) (layer "F.Cu") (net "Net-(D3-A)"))
 (segment (start 151.265 47.925) (end 151 48.19) (width 0.2) (layer "F.Cu") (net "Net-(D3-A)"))
 (segment (start 100.462564 83.610989) (end 101.034779 83.038774) (width 0.2) (layer "F.Cu") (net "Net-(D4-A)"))
 (segment (start 95.433825 83.610989) (end 100.462564 83.610989) (width 0.2) (layer "F.Cu") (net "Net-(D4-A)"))
 (segment (start 117.551249 142.513965) (end 118.737829 141.327385) (width 0.2) (layer "F.Cu") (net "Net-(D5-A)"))
 (segment (start 117.551249 146.831034) (end 117.551249 142.513965) (width 0.2) (layer "F.Cu") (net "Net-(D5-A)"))
 (segment (start 187.239462 142.604464) (end 184.511744 145.332182) (width 0.2) (layer "F.Cu") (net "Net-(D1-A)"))
 (segment (start 187.239462 137.082355) (end 187.239462 142.604464) (width 0.2) (layer "F.Cu") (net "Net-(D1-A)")))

